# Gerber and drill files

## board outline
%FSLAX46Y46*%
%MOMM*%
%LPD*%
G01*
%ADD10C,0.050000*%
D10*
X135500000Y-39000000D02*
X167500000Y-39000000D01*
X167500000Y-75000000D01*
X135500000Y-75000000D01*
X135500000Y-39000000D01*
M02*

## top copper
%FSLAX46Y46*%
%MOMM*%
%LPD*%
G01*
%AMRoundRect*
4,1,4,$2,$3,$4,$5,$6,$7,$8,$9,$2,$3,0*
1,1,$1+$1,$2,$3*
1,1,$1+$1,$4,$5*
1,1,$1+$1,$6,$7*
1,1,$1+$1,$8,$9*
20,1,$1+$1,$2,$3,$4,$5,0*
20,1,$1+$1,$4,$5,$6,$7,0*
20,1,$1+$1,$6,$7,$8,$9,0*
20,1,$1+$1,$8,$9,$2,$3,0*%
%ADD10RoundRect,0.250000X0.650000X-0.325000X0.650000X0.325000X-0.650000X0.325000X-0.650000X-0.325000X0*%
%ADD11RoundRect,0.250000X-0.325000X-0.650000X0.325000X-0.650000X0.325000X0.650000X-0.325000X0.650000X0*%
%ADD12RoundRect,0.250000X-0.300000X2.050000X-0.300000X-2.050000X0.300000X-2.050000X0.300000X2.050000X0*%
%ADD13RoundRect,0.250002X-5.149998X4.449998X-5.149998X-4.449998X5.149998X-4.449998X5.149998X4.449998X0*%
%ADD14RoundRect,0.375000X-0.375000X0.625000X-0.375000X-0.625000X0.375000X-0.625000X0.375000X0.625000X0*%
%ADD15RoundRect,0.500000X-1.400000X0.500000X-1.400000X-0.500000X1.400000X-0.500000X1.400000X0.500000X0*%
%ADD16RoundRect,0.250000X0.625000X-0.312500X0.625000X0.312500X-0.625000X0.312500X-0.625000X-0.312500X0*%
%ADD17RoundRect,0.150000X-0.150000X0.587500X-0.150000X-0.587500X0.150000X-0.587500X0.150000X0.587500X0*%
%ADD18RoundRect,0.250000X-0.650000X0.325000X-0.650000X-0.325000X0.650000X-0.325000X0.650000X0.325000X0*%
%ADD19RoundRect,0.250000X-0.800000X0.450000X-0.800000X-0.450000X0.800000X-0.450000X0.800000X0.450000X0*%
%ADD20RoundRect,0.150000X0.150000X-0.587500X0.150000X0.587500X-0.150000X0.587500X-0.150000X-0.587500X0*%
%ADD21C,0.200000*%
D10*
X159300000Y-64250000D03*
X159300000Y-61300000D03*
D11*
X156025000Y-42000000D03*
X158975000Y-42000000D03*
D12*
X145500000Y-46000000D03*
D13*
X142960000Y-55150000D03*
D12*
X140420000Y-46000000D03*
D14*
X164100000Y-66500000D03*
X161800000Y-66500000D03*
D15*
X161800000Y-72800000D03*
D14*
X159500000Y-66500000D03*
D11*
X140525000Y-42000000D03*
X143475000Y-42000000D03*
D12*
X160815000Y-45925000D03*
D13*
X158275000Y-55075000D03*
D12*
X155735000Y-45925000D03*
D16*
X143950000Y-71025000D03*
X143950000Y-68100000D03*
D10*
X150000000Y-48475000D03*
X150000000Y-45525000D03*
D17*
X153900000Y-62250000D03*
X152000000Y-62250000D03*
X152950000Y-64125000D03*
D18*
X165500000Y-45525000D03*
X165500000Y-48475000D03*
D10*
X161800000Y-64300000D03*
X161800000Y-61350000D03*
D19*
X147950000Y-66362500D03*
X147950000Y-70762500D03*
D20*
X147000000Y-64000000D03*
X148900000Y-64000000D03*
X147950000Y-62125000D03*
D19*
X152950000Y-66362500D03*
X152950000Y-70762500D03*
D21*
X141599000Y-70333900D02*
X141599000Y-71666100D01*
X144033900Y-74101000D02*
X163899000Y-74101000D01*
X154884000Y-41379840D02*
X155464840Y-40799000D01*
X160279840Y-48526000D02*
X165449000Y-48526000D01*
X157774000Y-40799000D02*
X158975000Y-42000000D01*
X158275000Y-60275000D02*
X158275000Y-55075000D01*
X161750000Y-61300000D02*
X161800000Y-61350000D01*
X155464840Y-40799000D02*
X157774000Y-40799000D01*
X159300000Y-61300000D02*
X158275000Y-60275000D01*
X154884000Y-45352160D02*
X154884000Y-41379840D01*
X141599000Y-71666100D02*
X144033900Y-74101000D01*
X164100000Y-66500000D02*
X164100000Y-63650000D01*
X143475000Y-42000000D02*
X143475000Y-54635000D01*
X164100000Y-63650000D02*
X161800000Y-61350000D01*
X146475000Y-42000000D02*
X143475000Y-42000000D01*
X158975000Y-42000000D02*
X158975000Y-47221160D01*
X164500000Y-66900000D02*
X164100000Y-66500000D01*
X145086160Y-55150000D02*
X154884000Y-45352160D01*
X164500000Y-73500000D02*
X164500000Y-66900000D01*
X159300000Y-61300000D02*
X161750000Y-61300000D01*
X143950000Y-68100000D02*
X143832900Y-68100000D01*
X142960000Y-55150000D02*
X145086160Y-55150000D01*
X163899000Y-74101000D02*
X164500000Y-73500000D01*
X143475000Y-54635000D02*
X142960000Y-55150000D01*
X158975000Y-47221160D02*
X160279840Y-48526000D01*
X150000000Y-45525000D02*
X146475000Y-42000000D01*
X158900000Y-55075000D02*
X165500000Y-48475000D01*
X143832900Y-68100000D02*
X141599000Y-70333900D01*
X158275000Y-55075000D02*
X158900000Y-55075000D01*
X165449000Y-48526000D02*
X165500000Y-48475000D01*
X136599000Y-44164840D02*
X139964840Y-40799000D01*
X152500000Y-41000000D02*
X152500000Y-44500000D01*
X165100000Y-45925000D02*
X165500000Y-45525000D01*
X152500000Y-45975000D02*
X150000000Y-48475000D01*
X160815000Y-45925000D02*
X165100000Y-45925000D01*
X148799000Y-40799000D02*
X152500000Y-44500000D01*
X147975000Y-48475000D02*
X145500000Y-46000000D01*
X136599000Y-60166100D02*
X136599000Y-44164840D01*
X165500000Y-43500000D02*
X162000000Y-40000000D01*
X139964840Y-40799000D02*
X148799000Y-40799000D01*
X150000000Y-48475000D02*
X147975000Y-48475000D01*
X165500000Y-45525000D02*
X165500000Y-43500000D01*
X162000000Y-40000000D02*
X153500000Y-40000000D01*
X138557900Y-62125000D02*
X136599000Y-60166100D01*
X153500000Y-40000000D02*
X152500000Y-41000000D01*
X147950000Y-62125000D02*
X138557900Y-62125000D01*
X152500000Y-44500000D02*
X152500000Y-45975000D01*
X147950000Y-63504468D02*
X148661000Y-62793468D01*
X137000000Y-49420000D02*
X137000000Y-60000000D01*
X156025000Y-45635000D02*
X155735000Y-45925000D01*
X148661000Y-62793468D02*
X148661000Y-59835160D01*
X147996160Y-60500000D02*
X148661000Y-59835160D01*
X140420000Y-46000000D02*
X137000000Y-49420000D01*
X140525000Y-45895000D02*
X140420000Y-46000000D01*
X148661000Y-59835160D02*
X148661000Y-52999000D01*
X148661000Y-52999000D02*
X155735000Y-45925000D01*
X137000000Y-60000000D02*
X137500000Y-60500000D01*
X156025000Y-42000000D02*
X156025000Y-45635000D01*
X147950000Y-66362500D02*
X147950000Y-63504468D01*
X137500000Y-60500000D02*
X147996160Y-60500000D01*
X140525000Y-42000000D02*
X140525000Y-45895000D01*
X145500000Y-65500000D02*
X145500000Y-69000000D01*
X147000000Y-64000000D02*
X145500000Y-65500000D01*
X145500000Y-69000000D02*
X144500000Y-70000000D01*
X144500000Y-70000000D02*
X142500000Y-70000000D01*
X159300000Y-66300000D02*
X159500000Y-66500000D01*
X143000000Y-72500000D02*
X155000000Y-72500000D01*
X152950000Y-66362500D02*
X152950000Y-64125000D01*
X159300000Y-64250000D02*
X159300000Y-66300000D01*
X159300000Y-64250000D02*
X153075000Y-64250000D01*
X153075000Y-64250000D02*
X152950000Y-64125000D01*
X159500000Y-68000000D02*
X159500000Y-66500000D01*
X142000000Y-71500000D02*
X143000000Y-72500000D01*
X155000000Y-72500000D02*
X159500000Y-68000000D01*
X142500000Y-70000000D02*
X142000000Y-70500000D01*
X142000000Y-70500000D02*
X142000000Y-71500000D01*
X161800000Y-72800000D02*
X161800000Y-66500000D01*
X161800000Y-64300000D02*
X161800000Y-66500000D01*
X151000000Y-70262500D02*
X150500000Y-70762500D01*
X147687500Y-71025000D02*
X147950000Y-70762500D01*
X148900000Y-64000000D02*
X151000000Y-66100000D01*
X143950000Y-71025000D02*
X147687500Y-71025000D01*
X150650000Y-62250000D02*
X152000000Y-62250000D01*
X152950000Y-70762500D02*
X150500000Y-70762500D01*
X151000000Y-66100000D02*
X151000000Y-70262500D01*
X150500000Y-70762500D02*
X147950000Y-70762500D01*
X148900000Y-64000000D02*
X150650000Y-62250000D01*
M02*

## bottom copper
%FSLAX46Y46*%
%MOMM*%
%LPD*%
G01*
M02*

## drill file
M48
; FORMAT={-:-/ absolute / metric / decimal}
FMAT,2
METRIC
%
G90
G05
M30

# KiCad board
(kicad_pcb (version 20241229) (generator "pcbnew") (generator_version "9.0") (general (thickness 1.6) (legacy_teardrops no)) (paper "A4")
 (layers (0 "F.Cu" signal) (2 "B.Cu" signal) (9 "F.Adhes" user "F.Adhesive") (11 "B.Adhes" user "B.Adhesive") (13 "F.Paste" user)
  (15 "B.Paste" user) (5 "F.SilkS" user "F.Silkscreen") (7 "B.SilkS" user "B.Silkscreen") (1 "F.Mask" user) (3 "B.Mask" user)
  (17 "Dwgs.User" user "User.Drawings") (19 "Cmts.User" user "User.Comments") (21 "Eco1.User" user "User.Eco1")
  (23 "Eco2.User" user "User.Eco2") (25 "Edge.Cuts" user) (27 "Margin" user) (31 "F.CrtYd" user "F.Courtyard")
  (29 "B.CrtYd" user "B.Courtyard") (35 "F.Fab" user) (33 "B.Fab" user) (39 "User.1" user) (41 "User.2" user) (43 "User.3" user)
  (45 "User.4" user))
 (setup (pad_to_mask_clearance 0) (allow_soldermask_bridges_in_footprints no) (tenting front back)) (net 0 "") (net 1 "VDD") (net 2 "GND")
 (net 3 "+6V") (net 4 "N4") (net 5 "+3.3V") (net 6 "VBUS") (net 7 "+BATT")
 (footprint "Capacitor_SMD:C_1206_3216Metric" (layer "F.Cu") (at 159.3 62.775 90)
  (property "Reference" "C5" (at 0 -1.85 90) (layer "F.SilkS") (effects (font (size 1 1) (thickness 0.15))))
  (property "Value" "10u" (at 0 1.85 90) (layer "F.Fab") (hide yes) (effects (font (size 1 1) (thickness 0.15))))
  (pad "1" smd roundrect (at -1.475 0 90) (size 1.15 1.8) (layers "F.Cu" "F.Mask" "F.Paste") (roundrect_rratio 0.217391) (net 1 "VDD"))
  (pad "2" smd roundrect (at 1.475 0 90) (size 1.15 1.8) (layers "F.Cu" "F.Mask" "F.Paste") (roundrect_rratio 0.217391) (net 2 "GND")))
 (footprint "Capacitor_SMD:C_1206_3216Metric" (layer "F.Cu") (at 157.5 42)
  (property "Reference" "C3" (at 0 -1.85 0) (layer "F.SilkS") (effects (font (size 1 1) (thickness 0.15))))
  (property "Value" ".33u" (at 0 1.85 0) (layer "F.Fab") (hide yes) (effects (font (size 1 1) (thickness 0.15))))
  (pad "1" smd roundrect (at -1.475 0) (size 1.15 1.8) (layers "F.Cu" "F.Mask" "F.Paste") (roundrect_rratio 0.217391) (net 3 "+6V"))
  (pad "2" smd roundrect (at 1.475 0) (size 1.15 1.8) (layers "F.Cu" "F.Mask" "F.Paste") (roundrect_rratio 0.217391) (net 2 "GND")))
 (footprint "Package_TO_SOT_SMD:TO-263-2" (layer "F.Cu") (at 142.96 53.65 -90)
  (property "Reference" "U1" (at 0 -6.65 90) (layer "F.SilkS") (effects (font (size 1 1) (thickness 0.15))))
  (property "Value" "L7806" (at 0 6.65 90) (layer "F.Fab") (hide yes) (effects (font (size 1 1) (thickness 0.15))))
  (pad "" smd roundrect (at -0.925 -2.775 270) (size 4.55 5.25) (layers "F.Paste") (roundrect_rratio 0.054945))
  (pad "" smd roundrect (at -0.925 2.775 270) (size 4.55 5.25) (layers "F.Paste") (roundrect_rratio 0.054945))
  (pad "" smd roundrect (at 3.925 -2.775 270) (size 4.55 5.25) (layers "F.Paste") (roundrect_rratio 0.054945))
  (pad "" smd roundrect (at 3.925 2.775 270) (size 4.55 5.25) (layers "F.Paste") (roundrect_rratio 0.054945))
  (pad "1" smd roundrect (at -7.65 -2.54 270) (size 4.6 1.1) (layers "F.Cu" "F.Mask" "F.Paste") (roundrect_rratio 0.227273) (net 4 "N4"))
  (pad "2" smd roundrect (at 1.5 0 270) (size 9.4 10.8) (layers "F.Cu" "F.Mask") (roundrect_rratio 0.026596) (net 2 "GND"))
  (pad "3" smd roundrect (at -7.65 2.54 270) (size 4.6 1.1) (layers "F.Cu" "F.Mask" "F.Paste") (roundrect_rratio 0.227273) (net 3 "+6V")))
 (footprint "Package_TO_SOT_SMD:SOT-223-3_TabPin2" (layer "F.Cu") (at 161.8 69.65 -90)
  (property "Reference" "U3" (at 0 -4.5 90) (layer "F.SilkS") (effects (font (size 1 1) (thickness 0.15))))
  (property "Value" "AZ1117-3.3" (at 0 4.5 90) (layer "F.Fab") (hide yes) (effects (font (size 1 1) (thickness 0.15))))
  (pad "1" smd roundrect (at -3.15 -2.3 270) (size 2 1.5) (layers "F.Cu" "F.Mask" "F.Paste") (roundrect_rratio 0.25) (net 2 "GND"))
  (pad "2" smd roundrect (at -3.15 0 270) (size 2 1.5) (layers "F.Cu" "F.Mask" "F.Paste") (roundrect_rratio 0.25) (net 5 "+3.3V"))
  (pad "2" smd roundrect (at 3.15 0 270) (size 2 3.8) (layers "F.Cu" "F.Mask" "F.Paste") (roundrect_rratio 0.25) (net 5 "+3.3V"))
  (pad "3" smd roundrect (at -3.15 2.3 270) (size 2 1.5) (layers "F.Cu" "F.Mask" "F.Paste") (roundrect_rratio 0.25) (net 1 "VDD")))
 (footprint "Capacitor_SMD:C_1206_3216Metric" (layer "F.Cu") (at 142 42)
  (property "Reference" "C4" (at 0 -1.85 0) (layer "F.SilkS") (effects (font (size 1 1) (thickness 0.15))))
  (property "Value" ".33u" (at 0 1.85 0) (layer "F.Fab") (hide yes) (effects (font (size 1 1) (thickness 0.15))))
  (pad "1" smd roundrect (at -1.475 0) (size 1.15 1.8) (layers "F.Cu" "F.Mask" "F.Paste") (roundrect_rratio 0.217391) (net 3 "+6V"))
  (pad "2" smd roundrect (at 1.475 0) (size 1.15 1.8) (layers "F.Cu" "F.Mask" "F.Paste") (roundrect_rratio 0.217391) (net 2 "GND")))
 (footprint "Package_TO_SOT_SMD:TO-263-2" (layer "F.Cu") (at 158.275 53.575 -90)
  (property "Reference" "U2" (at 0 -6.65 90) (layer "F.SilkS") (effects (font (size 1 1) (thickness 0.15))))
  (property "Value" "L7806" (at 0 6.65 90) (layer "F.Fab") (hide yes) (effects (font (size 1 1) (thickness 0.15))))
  (pad "" smd roundrect (at -0.925 -2.775 270) (size 4.55 5.25) (layers "F.Paste") (roundrect_rratio 0.054945))
  (pad "" smd roundrect (at -0.925 2.775 270) (size 4.55 5.25) (layers "F.Paste") (roundrect_rratio 0.054945))
  (pad "" smd roundrect (at 3.925 -2.775 270) (size 4.55 5.25) (layers "F.Paste") (roundrect_rratio 0.054945))
  (pad "" smd roundrect (at 3.925 2.775 270) (size 4.55 5.25) (layers "F.Paste") (roundrect_rratio 0.054945))
  (pad "1" smd roundrect (at -7.65 -2.54 270) (size 4.6 1.1) (layers "F.Cu" "F.Mask" "F.Paste") (roundrect_rratio 0.227273) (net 4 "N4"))
  (pad "2" smd roundrect (at 1.5 0 270) (size 9.4 10.8) (layers "F.Cu" "F.Mask") (roundrect_rratio 0.026596) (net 2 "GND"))
  (pad "3" smd roundrect (at -7.65 2.54 270) (size 4.6 1.1) (layers "F.Cu" "F.Mask" "F.Paste") (roundrect_rratio 0.227273) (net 3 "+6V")))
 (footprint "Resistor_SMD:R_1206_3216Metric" (layer "F.Cu") (at 143.95 69.5625 90)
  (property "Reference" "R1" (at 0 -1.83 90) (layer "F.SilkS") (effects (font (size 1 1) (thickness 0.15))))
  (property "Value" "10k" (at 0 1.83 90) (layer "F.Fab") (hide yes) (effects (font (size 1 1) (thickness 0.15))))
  (pad "1" smd roundrect (at -1.4625 0 90) (size 1.125 1.75) (layers "F.Cu" "F.Mask" "F.Paste") (roundrect_rratio 0.222222) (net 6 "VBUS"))
  (pad "2" smd roundrect (at 1.4625 0 90) (size 1.125 1.75) (layers "F.Cu" "F.Mask" "F.Paste") (roundrect_rratio 0.222222) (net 2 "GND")))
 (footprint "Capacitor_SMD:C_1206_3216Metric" (layer "F.Cu") (at 150 47 90)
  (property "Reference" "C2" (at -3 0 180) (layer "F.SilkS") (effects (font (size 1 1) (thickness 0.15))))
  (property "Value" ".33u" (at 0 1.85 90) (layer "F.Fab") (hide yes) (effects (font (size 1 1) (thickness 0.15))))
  (pad "1" smd roundrect (at -1.475 0 90) (size 1.15 1.8) (layers "F.Cu" "F.Mask" "F.Paste") (roundrect_rratio 0.217391) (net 4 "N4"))
  (pad "2" smd roundrect (at 1.475 0 90) (size 1.15 1.8) (layers "F.Cu" "F.Mask" "F.Paste") (roundrect_rratio 0.217391) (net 2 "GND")))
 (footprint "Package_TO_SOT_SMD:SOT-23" (layer "F.Cu") (at 152.95 63.1875 -90)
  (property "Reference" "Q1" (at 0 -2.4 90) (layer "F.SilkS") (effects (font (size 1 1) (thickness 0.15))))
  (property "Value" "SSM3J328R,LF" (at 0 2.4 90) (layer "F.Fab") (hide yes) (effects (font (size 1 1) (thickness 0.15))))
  (pad "1" smd roundrect (at -0.9375 -0.95 270) (size 1.475 0.6) (layers "F.Cu" "F.Mask" "F.Paste") (roundrect_rratio 0.25) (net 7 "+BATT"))
  (pad "2" smd roundrect (at -0.9375 0.95 270) (size 1.475 0.6) (layers "F.Cu" "F.Mask" "F.Paste") (roundrect_rratio 0.25) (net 6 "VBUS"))
  (pad "3" smd roundrect (at 0.9375 0 270) (size 1.475 0.6) (layers "F.Cu" "F.Mask" "F.Paste") (roundrect_rratio 0.25) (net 1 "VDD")))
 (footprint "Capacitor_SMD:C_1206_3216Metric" (layer "F.Cu") (at 165.5 47 -90)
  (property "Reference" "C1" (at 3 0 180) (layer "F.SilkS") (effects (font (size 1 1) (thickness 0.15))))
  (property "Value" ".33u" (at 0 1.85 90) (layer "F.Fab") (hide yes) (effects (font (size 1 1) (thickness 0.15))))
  (pad "1" smd roundrect (at -1.475 0 270) (size 1.15 1.8) (layers "F.Cu" "F.Mask" "F.Paste") (roundrect_rratio 0.217391) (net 4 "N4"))
  (pad "2" smd roundrect (at 1.475 0 270) (size 1.15 1.8) (layers "F.Cu" "F.Mask" "F.Paste") (roundrect_rratio 0.217391) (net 2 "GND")))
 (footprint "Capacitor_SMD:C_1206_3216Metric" (layer "F.Cu") (at 161.8 62.825 90)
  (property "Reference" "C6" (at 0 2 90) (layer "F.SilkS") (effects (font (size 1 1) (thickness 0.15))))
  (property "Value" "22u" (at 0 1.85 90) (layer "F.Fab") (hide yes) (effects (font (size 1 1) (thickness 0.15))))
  (pad "1" smd roundrect (at -1.475 0 90) (size 1.15 1.8) (layers "F.Cu" "F.Mask" "F.Paste") (roundrect_rratio 0.217391) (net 5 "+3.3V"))
  (pad "2" smd roundrect (at 1.475 0 90) (size 1.15 1.8) (layers "F.Cu" "F.Mask" "F.Paste") (roundrect_rratio 0.217391) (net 2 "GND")))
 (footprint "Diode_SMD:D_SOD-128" (layer "F.Cu") (at 147.95 68.5625 -90)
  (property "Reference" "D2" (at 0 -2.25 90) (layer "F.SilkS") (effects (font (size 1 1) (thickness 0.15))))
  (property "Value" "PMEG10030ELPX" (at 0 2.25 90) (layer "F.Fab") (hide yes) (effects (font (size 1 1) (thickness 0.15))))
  (pad "1" smd roundrect (at -2.2 0 270) (size 1.4 2.1) (layers "F.Cu" "F.Mask" "F.Paste") (roundrect_rratio 0.1785714286) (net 3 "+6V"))
  (pad "2" smd roundrect (at 2.2 0 270) (size 1.4 2.1) (layers "F.Cu" "F.Mask" "F.Paste") (roundrect_rratio 0.1785714286) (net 6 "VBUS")))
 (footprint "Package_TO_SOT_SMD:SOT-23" (layer "F.Cu") (at 147.95 63.0625 90)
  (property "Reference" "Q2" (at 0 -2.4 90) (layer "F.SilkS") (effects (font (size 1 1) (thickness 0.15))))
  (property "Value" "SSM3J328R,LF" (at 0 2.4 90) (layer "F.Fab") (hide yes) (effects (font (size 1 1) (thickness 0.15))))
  (pad "1" smd roundrect (at -0.9375 -0.95 90) (size 1.475 0.6) (layers "F.Cu" "F.Mask" "F.Paste") (roundrect_rratio 0.25) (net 1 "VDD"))
  (pad "2" smd roundrect (at -0.9375 0.95 90) (size 1.475 0.6) (layers "F.Cu" "F.Mask" "F.Paste") (roundrect_rratio 0.25) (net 6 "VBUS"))
  (pad "3" smd roundrect (at 0.9375 0 90) (size 1.475 0.6) (layers "F.Cu" "F.Mask" "F.Paste") (roundrect_rratio 0.25) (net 4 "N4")))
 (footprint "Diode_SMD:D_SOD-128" (layer "F.Cu") (at 152.95 68.5625 -90)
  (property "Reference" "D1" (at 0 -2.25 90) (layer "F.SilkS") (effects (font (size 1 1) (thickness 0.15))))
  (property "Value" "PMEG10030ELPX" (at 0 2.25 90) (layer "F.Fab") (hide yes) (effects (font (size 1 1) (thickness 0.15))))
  (pad "1" smd roundrect (at -2.2 0 270) (size 1.4 2.1) (layers "F.Cu" "F.Mask" "F.Paste") (roundrect_rratio 0.1785714286) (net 1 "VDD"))
  (pad "2" smd roundrect (at 2.2 0 270) (size 1.4 2.1) (layers "F.Cu" "F.Mask" "F.Paste") (roundrect_rratio 0.1785714286) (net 6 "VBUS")))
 (gr_rect (start 135.5 39) (end 167.5 75) (stroke (width 0.05) (type default)) (fill no) (layer "Edge.Cuts"))
 (segment (start 141.599 70.3339) (end 141.599 71.6661) (width 0.2) (layer "F.Cu") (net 2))
 (segment (start 144.0339 74.101) (end 163.899 74.101) (width 0.2) (layer "F.Cu") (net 2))
 (segment (start 154.884 41.37984) (end 155.46484 40.799) (width 0.2) (layer "F.Cu") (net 2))
 (segment (start 160.27984 48.526) (end 165.449 48.526) (width 0.2) (layer "F.Cu") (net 2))
 (segment (start 157.774 40.799) (end 158.975 42) (width 0.2) (layer "F.Cu") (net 2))
 (segment (start 158.275 60.275) (end 158.275 55.075) (width 0.2) (layer "F.Cu") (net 2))
 (segment (start 161.75 61.3) (end 161.8 61.35) (width 0.2) (layer "F.Cu") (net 2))
 (segment (start 155.46484 40.799) (end 157.774 40.799) (width 0.2) (layer "F.Cu") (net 2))
 (segment (start 159.3 61.3) (end 158.275 60.275) (width 0.2) (layer "F.Cu") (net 2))
 (segment (start 154.884 45.35216) (end 154.884 41.37984) (width 0.2) (layer "F.Cu") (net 2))
 (segment (start 141.599 71.6661) (end 144.0339 74.101) (width 0.2) (layer "F.Cu") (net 2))
 (segment (start 164.1 66.5) (end 164.1 63.65) (width 0.2) (layer "F.Cu") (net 2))
 (segment (start 143.475 42) (end 143.475 54.635) (width 0.2) (layer "F.Cu") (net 2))
 (segment (start 164.1 63.65) (end 161.8 61.35) (width 0.2) (layer "F.Cu") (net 2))
 (segment (start 146.475 42) (end 143.475 42) (width 0.2) (layer "F.Cu") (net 2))
 (segment (start 158.975 42) (end 158.975 47.22116) (width 0.2) (layer "F.Cu") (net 2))
 (segment (start 164.5 66.9) (end 164.1 66.5) (width 0.2) (layer "F.Cu") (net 2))
 (segment (start 145.08616 55.15) (end 154.884 45.35216) (width 0.2) (layer "F.Cu") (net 2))
 (segment (start 164.5 73.5) (end 164.5 66.9) (width 0.2) (layer "F.Cu") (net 2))
 (segment (start 159.3 61.3) (end 161.75 61.3) (width 0.2) (layer "F.Cu") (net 2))
 (segment (start 143.95 68.1) (end 143.8329 68.1) (width 0.2) (layer "F.Cu") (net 2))
 (segment (start 142.96 55.15) (end 145.08616 55.15) (width 0.2) (layer "F.Cu") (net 2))
 (segment (start 163.899 74.101) (end 164.5 73.5) (width 0.2) (layer "F.Cu") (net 2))
 (segment (start 143.475 54.635) (end 142.96 55.15) (width 0.2) (layer "F.Cu") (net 2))
 (segment (start 158.975 47.22116) (end 160.27984 48.526) (width 0.2) (layer "F.Cu") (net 2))
 (segment (start 150 45.525) (end 146.475 42) (width 0.2) (layer "F.Cu") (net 2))
 (segment (start 158.9 55.075) (end 165.5 48.475) (width 0.2) (layer "F.Cu") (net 2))
 (segment (start 143.8329 68.1) (end 141.599 70.3339) (width 0.2) (layer "F.Cu") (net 2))
 (segment (start 158.275 55.075) (end 158.9 55.075) (width 0.2) (layer "F.Cu") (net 2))
 (segment (start 165.449 48.526) (end 165.5 48.475) (width 0.2) (layer "F.Cu") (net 2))
 (segment (start 136.599 44.16484) (end 139.96484 40.799) (width 0.2) (layer "F.Cu") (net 4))
 (segment (start 152.5 41) (end 152.5 44.5) (width 0.2) (layer "F.Cu") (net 4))
 (segment (start 165.1 45.925) (end 165.5 45.525) (width 0.2) (layer "F.Cu") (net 4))
 (segment (start 152.5 45.975) (end 150 48.475) (width 0.2) (layer "F.Cu") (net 4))
 (segment (start 160.815 45.925) (end 165.1 45.925) (width 0.2) (layer "F.Cu") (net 4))
 (segment (start 148.799 40.799) (end 152.5 44.5) (width 0.2) (layer "F.Cu") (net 4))
 (segment (start 147.975 48.475) (end 145.5 46) (width 0.2) (layer "F.Cu") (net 4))
 (segment (start 136.599 60.1661) (end 136.599 44.16484) (width 0.2) (layer "F.Cu") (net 4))
 (segment (start 165.5 43.5) (end 162 40) (width 0.2) (layer "F.Cu") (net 4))
 (segment (start 139.96484 40.799) (end 148.799 40.799) (width 0.2) (layer "F.Cu") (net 4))
 (segment (start 150 48.475) (end 147.975 48.475) (width 0.2) (layer "F.Cu") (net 4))
 (segment (start 165.5 45.525) (end 165.5 43.5) (width 0.2) (layer "F.Cu") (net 4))
 (segment (start 162 40) (end 153.5 40) (width 0.2) (layer "F.Cu") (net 4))
 (segment (start 138.5579 62.125) (end 136.599 60.1661) (width 0.2) (layer "F.Cu") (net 4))
 (segment (start 153.5 40) (end 152.5 41) (width 0.2) (layer "F.Cu") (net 4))
 (segment (start 147.95 62.125) (end 138.5579 62.125) (width 0.2) (layer "F.Cu") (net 4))
 (segment (start 152.5 44.5) (end 152.5 45.975) (width 0.2) (layer "F.Cu") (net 4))
 (segment (start 147.95 63.504468) (end 148.661 62.793468) (width 0.2) (layer "F.Cu") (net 3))
 (segment (start 137 49.42) (end 137 60) (width 0.2) (layer "F.Cu") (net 3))
 (segment (start 156.025 45.635) (end 155.735 45.925) (width 0.2) (layer "F.Cu") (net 3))
 (segment (start 148.661 62.793468) (end 148.661 59.83516) (width 0.2) (layer "F.Cu") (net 3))
 (segment (start 147.99616 60.5) (end 148.661 59.83516) (width 0.2) (layer "F.Cu") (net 3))
 (segment (start 140.42 46) (end 137 49.42) (width 0.2) (layer "F.Cu") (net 3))
 (segment (start 140.525 45.895) (end 140.42 46) (width 0.2) (layer "F.Cu") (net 3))
 (segment (start 148.661 59.83516) (end 148.661 52.999) (width 0.2) (layer "F.Cu") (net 3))
 (segment (start 148.661 52.999) (end 155.735 45.925) (width 0.2) (layer "F.Cu") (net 3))
 (segment (start 137 60) (end 137.5 60.5) (width 0.2) (layer "F.Cu") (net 3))
 (segment (start 156.025 42) (end 156.025 45.635) (width 0.2) (layer "F.Cu") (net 3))
 (segment (start 147.95 66.3625) (end 147.95 63.504468) (width 0.2) (layer "F.Cu") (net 3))
 (segment (start 137.5 60.5) (end 147.99616 60.5) (width 0.2) (layer "F.Cu") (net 3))
 (segment (start 140.525 42) (end 140.525 45.895) (width 0.2) (layer "F.Cu") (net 3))
 (segment (start 145.5 65.5) (end 145.5 69) (width 0.2) (layer "F.Cu") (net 1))
 (segment (start 147 64) (end 145.5 65.5) (width 0.2) (layer "F.Cu") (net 1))
 (segment (start 145.5 69) (end 144.5 70) (width 0.2) (layer "F.Cu") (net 1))
 (segment (start 144.5 70) (end 142.5 70) (width 0.2) (layer "F.Cu") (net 1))
 (segment (start 159.3 66.3) (end 159.5 66.5) (width 0.2) (layer "F.Cu") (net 1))
 (segment (start 143 72.5) (end 155 72.5) (width 0.2) (layer "F.Cu") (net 1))
 (segment (start 152.95 66.3625) (end 152.95 64.125) (width 0.2) (layer "F.Cu") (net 1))
 (segment (start 159.3 64.25) (end 159.3 66.3) (width 0.2) (layer "F.Cu") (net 1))
 (segment (start 159.3 64.25) (end 153.075 64.25) (width 0.2) (layer "F.Cu") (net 1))
 (segment (start 153.075 64.25) (end 152.95 64.125) (width 0.2) (layer "F.Cu") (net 1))
 (segment (start 159.5 68) (end 159.5 66.5) (width 0.2) (layer "F.Cu") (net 1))
 (segment (start 142 71.5) (end 143 72.5) (width 0.2) (layer "F.Cu") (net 1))
 (segment (start 155 72.5) (end 159.5 68) (width 0.2) (layer "F.Cu") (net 1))
 (segment (start 142.5 70) (end 142 70.5) (width 0.2) (layer "F.Cu") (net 1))
 (segment (start 142 70.5) (end 142 71.5) (width 0.2) (layer "F.Cu") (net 1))
 (segment (start 161.8 72.8) (end 161.8 66.5) (width 0.2) (layer "F.Cu") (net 5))
 (segment (start 161.8 64.3) (end 161.8 66.5) (width 0.2) (layer "F.Cu") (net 5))
 (segment (start 151 70.2625) (end 150.5 70.7625) (width 0.2) (layer "F.Cu") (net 6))
 (segment (start 147.6875 71.025) (end 147.95 70.7625) (width 0.2) (layer "F.Cu") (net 6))
 (segment (start 148.9 64) (end 151 66.1) (width 0.2) (layer "F.Cu") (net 6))
 (segment (start 143.95 71.025) (end 147.6875 71.025) (width 0.2) (layer "F.Cu") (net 6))
 (segment (start 150.65 62.25) (end 152 62.25) (width 0.2) (layer "F.Cu") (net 6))
 (segment (start 152.95 70.7625) (end 150.5 70.7625) (width 0.2) (layer "F.Cu") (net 6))
 (segment (start 151 66.1) (end 151 70.2625) (width 0.2) (layer "F.Cu") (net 6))
 (segment (start 150.5 70.7625) (end 147.95 70.7625) (width 0.2) (layer "F.Cu") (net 6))
 (segment (start 148.9 64) (end 150.65 62.25) (width 0.2) (layer "F.Cu") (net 6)))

